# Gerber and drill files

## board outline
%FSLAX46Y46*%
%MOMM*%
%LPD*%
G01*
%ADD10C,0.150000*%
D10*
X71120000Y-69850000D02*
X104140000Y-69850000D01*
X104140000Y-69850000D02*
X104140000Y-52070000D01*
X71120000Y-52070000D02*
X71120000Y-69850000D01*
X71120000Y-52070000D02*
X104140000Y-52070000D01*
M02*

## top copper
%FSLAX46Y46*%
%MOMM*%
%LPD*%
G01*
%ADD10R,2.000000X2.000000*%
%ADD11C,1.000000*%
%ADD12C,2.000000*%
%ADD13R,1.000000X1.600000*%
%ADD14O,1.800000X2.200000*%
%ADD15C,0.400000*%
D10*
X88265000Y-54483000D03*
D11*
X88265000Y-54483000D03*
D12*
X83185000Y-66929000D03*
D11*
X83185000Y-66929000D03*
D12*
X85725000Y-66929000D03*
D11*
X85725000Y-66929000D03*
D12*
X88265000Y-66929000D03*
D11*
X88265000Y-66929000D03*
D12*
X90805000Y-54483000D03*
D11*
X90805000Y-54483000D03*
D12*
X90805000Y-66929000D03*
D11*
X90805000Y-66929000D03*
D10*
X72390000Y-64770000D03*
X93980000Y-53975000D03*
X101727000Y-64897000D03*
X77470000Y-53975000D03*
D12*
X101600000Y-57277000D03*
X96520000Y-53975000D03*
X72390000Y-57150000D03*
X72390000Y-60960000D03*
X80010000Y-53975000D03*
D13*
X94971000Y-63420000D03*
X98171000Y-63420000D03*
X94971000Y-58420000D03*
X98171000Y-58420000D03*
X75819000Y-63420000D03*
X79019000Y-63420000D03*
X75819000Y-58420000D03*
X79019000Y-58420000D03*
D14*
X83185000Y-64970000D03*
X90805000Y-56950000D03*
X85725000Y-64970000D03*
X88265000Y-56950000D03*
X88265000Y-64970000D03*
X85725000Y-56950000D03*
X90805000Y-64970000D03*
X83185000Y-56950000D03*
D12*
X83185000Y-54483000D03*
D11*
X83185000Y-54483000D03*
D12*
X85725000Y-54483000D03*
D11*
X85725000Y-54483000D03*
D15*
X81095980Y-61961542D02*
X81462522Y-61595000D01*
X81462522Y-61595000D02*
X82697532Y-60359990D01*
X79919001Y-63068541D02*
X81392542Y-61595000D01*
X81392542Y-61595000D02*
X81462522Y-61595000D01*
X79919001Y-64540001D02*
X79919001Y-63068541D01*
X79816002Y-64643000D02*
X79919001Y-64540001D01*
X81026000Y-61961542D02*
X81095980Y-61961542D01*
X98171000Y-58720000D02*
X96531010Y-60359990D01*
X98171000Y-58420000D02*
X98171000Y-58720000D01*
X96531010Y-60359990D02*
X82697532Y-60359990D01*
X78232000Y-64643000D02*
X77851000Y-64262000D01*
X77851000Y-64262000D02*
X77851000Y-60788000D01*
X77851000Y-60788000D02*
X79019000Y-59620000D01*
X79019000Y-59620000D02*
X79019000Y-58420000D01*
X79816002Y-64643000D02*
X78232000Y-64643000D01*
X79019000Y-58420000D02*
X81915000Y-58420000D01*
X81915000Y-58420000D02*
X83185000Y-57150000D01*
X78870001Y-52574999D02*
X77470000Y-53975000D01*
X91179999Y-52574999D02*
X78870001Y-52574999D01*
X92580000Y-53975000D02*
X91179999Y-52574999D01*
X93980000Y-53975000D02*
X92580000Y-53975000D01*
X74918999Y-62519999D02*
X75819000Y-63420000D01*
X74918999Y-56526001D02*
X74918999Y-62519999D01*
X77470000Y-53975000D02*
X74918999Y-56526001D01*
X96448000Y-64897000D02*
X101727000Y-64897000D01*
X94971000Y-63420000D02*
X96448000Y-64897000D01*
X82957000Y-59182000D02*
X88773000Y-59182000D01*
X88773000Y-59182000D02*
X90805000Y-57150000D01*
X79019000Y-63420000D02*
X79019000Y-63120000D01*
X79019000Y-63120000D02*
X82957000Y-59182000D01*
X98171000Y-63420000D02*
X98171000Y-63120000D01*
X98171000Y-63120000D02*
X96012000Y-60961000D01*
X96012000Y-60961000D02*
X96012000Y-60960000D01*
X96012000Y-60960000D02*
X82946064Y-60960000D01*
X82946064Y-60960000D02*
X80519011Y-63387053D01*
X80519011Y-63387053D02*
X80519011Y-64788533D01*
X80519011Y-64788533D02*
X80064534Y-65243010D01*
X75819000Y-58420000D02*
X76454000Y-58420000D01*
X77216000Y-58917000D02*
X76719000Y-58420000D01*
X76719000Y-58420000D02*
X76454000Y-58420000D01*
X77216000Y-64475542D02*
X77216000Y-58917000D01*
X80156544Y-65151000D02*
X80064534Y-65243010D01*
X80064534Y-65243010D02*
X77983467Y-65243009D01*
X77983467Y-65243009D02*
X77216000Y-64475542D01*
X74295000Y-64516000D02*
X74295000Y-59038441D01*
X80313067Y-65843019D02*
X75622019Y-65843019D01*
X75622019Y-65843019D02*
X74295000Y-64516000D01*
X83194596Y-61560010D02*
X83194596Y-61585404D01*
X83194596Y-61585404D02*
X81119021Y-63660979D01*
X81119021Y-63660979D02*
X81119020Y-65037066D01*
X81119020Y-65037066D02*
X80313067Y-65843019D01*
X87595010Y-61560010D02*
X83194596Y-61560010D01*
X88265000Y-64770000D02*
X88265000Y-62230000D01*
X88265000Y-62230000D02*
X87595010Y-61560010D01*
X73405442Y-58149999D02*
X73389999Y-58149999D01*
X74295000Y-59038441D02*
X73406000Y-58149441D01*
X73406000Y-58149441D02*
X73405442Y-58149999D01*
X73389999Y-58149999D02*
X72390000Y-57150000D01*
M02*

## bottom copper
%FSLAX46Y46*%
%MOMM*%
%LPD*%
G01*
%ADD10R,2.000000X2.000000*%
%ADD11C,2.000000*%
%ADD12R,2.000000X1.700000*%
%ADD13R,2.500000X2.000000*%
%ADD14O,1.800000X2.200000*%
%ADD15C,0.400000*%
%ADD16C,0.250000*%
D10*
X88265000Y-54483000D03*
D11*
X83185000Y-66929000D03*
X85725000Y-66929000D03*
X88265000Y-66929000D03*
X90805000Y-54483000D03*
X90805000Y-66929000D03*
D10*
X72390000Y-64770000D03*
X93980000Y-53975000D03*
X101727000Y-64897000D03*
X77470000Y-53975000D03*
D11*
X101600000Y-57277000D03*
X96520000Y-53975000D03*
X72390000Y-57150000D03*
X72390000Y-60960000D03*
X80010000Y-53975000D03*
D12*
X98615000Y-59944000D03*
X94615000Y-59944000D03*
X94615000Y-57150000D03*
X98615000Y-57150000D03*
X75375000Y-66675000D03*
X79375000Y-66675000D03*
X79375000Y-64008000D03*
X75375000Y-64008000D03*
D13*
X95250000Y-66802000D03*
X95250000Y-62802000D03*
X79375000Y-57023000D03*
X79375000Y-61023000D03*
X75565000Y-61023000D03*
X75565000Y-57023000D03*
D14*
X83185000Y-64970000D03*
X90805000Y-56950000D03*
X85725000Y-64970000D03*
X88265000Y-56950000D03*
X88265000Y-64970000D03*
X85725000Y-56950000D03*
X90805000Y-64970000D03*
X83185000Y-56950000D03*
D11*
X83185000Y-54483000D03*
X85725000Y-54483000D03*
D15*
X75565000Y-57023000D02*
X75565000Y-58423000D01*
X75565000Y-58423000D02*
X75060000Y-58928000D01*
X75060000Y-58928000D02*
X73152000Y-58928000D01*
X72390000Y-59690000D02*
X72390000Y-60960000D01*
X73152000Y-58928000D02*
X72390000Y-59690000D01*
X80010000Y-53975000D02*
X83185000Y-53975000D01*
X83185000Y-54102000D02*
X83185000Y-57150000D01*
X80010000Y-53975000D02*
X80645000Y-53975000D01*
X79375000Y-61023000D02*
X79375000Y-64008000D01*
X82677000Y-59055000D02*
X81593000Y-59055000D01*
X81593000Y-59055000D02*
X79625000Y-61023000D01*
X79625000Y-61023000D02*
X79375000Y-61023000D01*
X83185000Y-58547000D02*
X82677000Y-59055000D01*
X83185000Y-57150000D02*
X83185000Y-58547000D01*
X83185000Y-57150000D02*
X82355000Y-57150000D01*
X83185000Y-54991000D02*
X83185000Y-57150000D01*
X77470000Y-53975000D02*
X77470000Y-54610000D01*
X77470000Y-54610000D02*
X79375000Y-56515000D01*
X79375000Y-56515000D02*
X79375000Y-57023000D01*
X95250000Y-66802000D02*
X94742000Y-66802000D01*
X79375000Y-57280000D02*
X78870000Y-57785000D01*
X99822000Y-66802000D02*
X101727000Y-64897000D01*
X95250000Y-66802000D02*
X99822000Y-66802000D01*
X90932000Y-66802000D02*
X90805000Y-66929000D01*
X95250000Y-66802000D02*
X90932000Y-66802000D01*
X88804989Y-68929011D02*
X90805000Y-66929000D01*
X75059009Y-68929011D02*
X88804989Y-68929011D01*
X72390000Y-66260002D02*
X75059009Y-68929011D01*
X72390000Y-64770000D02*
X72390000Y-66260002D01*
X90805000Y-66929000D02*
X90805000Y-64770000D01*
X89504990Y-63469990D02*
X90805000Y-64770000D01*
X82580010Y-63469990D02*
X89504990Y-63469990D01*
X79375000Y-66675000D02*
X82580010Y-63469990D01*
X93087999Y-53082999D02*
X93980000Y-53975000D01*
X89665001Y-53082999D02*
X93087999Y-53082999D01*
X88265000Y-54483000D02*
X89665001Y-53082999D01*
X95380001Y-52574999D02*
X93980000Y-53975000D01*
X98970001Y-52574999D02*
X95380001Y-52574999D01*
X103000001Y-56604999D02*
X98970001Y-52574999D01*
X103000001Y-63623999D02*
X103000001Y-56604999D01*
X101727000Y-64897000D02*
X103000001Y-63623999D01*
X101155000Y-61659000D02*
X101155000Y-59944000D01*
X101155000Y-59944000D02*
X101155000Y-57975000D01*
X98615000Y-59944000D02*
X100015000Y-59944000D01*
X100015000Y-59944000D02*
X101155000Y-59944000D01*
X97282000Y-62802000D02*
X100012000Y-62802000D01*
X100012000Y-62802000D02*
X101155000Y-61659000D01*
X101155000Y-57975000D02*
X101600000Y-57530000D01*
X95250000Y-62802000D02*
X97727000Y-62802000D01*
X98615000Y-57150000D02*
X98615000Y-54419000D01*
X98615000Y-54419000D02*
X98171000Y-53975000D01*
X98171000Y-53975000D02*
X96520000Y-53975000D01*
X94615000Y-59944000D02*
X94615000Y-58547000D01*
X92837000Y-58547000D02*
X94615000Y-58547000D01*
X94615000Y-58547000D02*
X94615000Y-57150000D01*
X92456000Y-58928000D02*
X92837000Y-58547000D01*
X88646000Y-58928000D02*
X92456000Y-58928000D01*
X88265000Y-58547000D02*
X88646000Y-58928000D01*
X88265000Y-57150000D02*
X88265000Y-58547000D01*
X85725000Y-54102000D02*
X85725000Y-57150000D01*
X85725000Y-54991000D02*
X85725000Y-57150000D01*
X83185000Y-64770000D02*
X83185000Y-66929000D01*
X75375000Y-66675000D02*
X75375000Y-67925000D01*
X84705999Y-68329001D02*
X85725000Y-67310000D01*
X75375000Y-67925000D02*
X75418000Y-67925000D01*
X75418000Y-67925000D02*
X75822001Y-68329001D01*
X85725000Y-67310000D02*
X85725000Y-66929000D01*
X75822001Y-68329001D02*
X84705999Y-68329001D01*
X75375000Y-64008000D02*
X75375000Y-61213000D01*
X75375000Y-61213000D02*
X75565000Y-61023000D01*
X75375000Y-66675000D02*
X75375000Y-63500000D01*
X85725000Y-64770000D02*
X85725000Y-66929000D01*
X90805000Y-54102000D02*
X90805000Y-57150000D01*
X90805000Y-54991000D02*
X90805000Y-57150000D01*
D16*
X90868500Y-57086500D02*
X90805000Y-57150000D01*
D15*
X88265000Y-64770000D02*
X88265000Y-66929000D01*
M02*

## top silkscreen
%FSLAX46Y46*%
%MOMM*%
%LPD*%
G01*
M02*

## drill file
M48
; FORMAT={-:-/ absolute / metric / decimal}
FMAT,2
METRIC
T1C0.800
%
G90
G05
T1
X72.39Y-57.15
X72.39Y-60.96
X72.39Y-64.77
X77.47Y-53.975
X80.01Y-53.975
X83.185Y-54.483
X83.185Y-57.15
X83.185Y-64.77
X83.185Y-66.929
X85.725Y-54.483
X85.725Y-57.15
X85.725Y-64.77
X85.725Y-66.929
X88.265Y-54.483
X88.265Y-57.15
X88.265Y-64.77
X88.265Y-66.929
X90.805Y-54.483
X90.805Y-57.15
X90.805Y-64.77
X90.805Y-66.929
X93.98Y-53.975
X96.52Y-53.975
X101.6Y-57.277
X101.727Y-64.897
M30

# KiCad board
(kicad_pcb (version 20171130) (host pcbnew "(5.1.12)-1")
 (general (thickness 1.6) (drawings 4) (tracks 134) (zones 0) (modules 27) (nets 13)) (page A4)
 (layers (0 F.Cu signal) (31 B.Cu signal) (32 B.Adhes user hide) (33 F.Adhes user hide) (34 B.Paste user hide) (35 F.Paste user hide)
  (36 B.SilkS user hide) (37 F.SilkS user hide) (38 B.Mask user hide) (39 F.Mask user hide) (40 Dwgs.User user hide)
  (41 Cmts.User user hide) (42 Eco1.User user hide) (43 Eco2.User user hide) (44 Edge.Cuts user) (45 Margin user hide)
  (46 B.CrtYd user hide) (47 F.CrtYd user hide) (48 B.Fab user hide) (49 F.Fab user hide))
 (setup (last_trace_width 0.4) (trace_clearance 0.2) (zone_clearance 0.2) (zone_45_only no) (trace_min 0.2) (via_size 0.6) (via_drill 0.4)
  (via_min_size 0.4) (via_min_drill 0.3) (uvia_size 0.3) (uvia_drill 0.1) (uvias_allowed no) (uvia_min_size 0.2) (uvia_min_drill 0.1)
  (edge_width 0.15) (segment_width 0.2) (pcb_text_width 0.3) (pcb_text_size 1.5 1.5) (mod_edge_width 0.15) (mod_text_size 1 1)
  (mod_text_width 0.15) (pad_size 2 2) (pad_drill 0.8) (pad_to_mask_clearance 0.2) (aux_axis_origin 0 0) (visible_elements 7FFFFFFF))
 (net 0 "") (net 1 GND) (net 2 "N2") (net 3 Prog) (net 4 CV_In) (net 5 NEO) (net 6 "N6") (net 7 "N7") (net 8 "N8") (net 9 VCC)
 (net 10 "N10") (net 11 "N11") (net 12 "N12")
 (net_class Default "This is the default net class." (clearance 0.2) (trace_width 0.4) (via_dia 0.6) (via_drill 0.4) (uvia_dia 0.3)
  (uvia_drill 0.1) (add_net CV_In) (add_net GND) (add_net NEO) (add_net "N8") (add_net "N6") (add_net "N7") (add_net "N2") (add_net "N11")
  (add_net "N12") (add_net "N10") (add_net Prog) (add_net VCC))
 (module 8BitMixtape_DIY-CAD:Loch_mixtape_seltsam (layer F.Cu) (at 88.265 54.483)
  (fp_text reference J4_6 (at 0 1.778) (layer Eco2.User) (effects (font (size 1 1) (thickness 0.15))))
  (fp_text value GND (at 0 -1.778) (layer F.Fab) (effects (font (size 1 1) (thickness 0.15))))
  (pad 1 thru_hole rect (at 0 0) (size 2 2) (drill 0.8) (layers B.Cu B.Mask) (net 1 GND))
  (pad "" smd circle (at 0 0) (size 1 1) (layers F.Cu F.Paste F.Mask)))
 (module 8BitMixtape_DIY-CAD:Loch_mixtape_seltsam (layer F.Cu) (at 83.185 66.929)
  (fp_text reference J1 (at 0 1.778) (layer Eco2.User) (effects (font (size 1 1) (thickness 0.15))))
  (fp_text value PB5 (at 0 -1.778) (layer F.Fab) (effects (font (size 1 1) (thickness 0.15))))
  (pad 1 thru_hole circle (at 0 0) (size 2 2) (drill 0.8) (layers B.Cu B.Mask) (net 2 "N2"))
  (pad "" smd circle (at 0 0) (size 1 1) (layers F.Cu F.Paste F.Mask)))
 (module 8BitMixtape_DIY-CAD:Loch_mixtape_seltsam (layer F.Cu) (at 85.725 66.929)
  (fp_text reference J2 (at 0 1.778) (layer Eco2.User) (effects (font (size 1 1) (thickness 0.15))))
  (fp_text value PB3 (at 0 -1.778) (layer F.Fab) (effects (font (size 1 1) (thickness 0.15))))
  (pad 1 thru_hole circle (at 0 0) (size 2 2) (drill 0.8) (layers B.Cu B.Mask) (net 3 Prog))
  (pad "" smd circle (at 0 0) (size 1 1) (layers F.Cu F.Paste F.Mask)))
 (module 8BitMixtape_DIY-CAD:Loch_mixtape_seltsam (layer F.Cu) (at 88.265 66.929)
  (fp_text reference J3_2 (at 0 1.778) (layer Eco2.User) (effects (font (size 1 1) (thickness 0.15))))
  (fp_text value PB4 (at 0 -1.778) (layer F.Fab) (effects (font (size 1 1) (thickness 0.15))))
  (pad 1 thru_hole circle (at 0 0) (size 2 2) (drill 0.8) (layers B.Cu B.Mask) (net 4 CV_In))
  (pad "" smd circle (at 0 0) (size 1 1) (layers F.Cu F.Paste F.Mask)))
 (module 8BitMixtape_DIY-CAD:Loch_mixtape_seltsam (layer F.Cu) (at 90.805 54.483)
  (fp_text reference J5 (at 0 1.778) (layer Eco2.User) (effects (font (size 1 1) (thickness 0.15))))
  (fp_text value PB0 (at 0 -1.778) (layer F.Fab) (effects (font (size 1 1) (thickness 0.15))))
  (pad 1 thru_hole circle (at 0 0) (size 2 2) (drill 0.8) (layers B.Cu B.Mask) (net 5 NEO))
  (pad "" smd circle (at 0 0) (size 1 1) (layers F.Cu F.Paste F.Mask)))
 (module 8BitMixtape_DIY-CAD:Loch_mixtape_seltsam (layer F.Cu) (at 90.805 66.929)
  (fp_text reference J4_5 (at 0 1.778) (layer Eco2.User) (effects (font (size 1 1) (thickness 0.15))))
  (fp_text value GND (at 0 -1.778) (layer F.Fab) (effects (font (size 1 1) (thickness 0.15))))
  (pad 1 thru_hole circle (at 0 0) (size 2 2) (drill 0.8) (layers B.Cu B.Mask) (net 1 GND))
  (pad "" smd circle (at 0 0) (size 1 1) (layers F.Cu F.Paste F.Mask)))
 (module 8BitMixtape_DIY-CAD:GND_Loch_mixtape (layer F.Cu) (at 72.39 64.77)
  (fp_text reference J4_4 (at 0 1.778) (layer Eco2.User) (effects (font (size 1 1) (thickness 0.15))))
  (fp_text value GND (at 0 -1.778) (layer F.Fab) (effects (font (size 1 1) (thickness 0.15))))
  (pad 1 thru_hole rect (at 0 0) (size 2 2) (drill 0.8) (layers *.Cu *.Mask) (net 1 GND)))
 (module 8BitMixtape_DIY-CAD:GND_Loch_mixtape (layer F.Cu) (at 93.98 53.975)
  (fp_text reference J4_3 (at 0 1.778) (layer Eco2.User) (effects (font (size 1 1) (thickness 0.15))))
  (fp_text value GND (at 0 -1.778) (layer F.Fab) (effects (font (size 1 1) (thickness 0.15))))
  (pad 1 thru_hole rect (at 0 0) (size 2 2) (drill 0.8) (layers *.Cu *.Mask) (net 1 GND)))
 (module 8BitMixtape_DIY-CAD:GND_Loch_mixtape (layer F.Cu) (at 101.727 64.897)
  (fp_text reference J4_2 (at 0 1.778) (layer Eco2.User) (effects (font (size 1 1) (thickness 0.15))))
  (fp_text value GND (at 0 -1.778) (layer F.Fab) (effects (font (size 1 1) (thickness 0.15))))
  (pad 1 thru_hole rect (at 0 0) (size 2 2) (drill 0.8) (layers *.Cu *.Mask) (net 1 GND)))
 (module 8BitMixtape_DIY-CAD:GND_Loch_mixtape (layer F.Cu) (at 77.47 53.975)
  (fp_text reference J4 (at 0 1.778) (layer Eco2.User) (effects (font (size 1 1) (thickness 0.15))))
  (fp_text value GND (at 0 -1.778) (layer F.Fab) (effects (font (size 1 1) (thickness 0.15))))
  (pad 1 thru_hole rect (at 0 0) (size 2 2) (drill 0.8) (layers *.Cu *.Mask) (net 1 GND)))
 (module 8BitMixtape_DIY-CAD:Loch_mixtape (layer F.Cu) (at 101.6 57.277)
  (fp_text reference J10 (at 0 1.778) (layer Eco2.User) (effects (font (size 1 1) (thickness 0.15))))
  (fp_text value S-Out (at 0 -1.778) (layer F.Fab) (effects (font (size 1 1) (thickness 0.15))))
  (pad 1 thru_hole circle (at 0 0) (size 2 2) (drill 0.8) (layers *.Cu *.Mask) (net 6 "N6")))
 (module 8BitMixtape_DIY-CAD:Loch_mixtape (layer F.Cu) (at 96.52 53.975)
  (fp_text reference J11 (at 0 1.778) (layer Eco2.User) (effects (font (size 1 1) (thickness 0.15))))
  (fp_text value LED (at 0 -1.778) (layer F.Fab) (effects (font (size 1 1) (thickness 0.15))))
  (pad 1 thru_hole circle (at 0 0) (size 2 2) (drill 0.8) (layers *.Cu *.Mask) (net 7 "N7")))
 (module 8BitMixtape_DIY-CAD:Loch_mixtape (layer F.Cu) (at 72.39 57.15)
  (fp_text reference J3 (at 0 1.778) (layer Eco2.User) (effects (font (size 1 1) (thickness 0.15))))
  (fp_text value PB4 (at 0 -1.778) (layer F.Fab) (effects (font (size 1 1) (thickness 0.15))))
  (pad 1 thru_hole circle (at 0 0) (size 2 2) (drill 0.8) (layers *.Cu *.Mask) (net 4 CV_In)))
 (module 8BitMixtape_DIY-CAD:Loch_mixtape (layer F.Cu) (at 72.39 60.96)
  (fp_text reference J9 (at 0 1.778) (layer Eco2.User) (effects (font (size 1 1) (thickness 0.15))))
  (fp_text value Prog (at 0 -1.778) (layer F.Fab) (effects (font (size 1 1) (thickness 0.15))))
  (pad 1 thru_hole circle (at 0 0) (size 2 2) (drill 0.8) (layers *.Cu *.Mask) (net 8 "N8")))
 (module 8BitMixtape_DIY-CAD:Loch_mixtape (layer F.Cu) (at 80.01 53.975)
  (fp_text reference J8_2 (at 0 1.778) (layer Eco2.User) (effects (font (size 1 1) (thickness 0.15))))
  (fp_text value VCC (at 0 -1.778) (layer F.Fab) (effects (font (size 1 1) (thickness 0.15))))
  (pad 1 thru_hole circle (at 0 0) (size 2 2) (drill 0.8) (layers *.Cu *.Mask) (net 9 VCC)))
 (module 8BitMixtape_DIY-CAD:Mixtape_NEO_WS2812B (layer F.Cu) (at 96.571 60.92 270)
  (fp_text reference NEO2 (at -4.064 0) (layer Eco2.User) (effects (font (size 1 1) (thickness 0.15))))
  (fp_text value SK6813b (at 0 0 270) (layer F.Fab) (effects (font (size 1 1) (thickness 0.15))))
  (pad 3 smd rect (at 2.5 1.6 270) (size 1.6 1) (layers F.Cu F.Paste F.Mask) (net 1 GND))
  (pad 4 smd rect (at 2.5 -1.6 270) (size 1.6 1) (layers F.Cu F.Paste F.Mask) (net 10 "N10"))
  (pad 2 smd rect (at -2.5 1.6 270) (size 1.6 1) (layers F.Cu F.Paste F.Mask))
  (pad 1 smd rect (at -2.5 -1.6 270) (size 1.6 1) (layers F.Cu F.Paste F.Mask) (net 9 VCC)))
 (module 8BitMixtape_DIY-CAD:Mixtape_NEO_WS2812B (layer F.Cu) (at 77.419 60.92 270)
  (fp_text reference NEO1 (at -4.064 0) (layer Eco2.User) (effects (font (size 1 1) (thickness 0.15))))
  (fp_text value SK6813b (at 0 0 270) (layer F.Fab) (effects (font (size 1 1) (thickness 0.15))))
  (pad 3 smd rect (at 2.5 1.6 270) (size 1.6 1) (layers F.Cu F.Paste F.Mask) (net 1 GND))
  (pad 4 smd rect (at 2.5 -1.6 270) (size 1.6 1) (layers F.Cu F.Paste F.Mask) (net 5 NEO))
  (pad 2 smd rect (at -2.5 1.6 270) (size 1.6 1) (layers F.Cu F.Paste F.Mask) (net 10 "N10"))
  (pad 1 smd rect (at -2.5 -1.6 270) (size 1.6 1) (layers F.Cu F.Paste F.Mask) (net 9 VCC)))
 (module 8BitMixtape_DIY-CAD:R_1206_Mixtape (layer B.Cu) (at 96.615 59.944 180)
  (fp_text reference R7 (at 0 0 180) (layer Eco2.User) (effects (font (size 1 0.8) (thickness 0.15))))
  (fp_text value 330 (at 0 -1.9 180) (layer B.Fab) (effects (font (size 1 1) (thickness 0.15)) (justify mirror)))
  (pad 1 smd rect (at -2 0 180) (size 2 1.7) (layers B.Cu B.Paste B.Mask) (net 6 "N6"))
  (pad 2 smd rect (at 2 0 180) (size 2 1.7) (layers B.Cu B.Paste B.Mask) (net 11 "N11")))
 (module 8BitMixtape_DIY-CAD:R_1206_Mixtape (layer B.Cu) (at 96.615 57.15)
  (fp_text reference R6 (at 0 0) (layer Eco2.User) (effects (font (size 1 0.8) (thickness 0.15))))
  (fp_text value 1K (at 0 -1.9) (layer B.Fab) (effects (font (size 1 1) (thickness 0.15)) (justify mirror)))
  (pad 1 smd rect (at -2 0) (size 2 1.7) (layers B.Cu B.Paste B.Mask) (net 11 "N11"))
  (pad 2 smd rect (at 2 0) (size 2 1.7) (layers B.Cu B.Paste B.Mask) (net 7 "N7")))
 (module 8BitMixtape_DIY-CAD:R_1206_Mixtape (layer B.Cu) (at 77.375 66.675)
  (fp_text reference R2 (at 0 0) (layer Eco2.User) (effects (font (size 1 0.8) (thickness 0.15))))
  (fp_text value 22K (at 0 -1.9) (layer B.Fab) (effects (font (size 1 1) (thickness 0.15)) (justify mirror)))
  (pad 1 smd rect (at -2 0) (size 2 1.7) (layers B.Cu B.Paste B.Mask) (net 3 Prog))
  (pad 2 smd rect (at 2 0) (size 2 1.7) (layers B.Cu B.Paste B.Mask) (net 1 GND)))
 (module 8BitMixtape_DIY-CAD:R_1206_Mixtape (layer B.Cu) (at 77.375 64.008 180)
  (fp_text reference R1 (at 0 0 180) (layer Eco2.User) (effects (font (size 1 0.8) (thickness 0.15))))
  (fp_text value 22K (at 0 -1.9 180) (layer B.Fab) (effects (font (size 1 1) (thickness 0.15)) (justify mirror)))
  (pad 1 smd rect (at -2 0 180) (size 2 1.7) (layers B.Cu B.Paste B.Mask) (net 9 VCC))
  (pad 2 smd rect (at 2 0 180) (size 2 1.7) (layers B.Cu B.Paste B.Mask) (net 3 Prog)))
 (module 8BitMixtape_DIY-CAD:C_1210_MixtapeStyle (layer B.Cu) (at 95.25 64.802 90)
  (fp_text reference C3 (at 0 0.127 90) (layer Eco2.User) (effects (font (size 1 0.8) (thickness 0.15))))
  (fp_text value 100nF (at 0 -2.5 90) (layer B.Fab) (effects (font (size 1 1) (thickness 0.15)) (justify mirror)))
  (pad 1 smd rect (at -2 0 90) (size 2 2.5) (layers B.Cu B.Paste B.Mask) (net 1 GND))
  (pad 2 smd rect (at 2 0 90) (size 2 2.5) (layers B.Cu B.Paste B.Mask) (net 6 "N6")))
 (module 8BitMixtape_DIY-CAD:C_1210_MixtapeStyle (layer B.Cu) (at 79.375 59.023 270)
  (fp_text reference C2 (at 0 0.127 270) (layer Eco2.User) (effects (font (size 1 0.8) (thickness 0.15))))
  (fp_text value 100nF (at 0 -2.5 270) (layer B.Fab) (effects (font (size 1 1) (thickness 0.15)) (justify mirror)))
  (pad 1 smd rect (at -2 0 270) (size 2 2.5) (layers B.Cu B.Paste B.Mask) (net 1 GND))
  (pad 2 smd rect (at 2 0 270) (size 2 2.5) (layers B.Cu B.Paste B.Mask) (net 9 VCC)))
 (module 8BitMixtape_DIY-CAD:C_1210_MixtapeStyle (layer B.Cu) (at 75.565 59.023 90)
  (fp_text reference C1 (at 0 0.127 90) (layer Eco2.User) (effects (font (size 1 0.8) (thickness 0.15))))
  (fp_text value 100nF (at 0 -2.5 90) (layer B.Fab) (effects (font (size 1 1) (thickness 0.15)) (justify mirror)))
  (pad 1 smd rect (at -2 0 90) (size 2 2.5) (layers B.Cu B.Paste B.Mask) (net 3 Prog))
  (pad 2 smd rect (at 2 0 90) (size 2 2.5) (layers B.Cu B.Paste B.Mask) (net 8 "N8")))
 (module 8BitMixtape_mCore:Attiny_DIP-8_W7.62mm (layer F.Cu) (at 83.185 64.77 90)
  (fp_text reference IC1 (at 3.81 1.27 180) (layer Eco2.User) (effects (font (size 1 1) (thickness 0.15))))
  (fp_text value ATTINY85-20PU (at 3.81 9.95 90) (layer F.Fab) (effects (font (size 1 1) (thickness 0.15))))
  (pad 1 thru_hole oval (at 0 0 90) (size 2.2 1.8) (drill 0.8 (offset -0.2 0)) (layers *.Cu *.Mask) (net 2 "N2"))
  (pad 5 thru_hole oval (at 7.62 7.62 90) (size 2.2 1.8) (drill 0.8 (offset 0.2 0)) (layers *.Cu *.Mask) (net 5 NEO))
  (pad 2 thru_hole oval (at 0 2.54 90) (size 2.2 1.8) (drill 0.8 (offset -0.2 0)) (layers *.Cu *.Mask) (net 3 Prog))
  (pad 6 thru_hole oval (at 7.62 5.08 90) (size 2.2 1.8) (drill 0.8 (offset 0.2 0)) (layers *.Cu *.Mask) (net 11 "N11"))
  (pad 3 thru_hole oval (at 0 5.08 90) (size 2.2 1.8) (drill 0.8 (offset -0.2 0)) (layers *.Cu *.Mask) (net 4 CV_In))
  (pad 7 thru_hole oval (at 7.62 2.54 90) (size 2.2 1.8) (drill 0.8 (offset 0.2 0)) (layers *.Cu *.Mask) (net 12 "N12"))
  (pad 4 thru_hole oval (at 0 7.62 90) (size 2.2 1.8) (drill 0.8 (offset -0.2 0)) (layers *.Cu *.Mask) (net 1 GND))
  (pad 8 thru_hole oval (at 7.62 0 90) (size 2.2 1.8) (drill 0.8 (offset 0.2 0)) (layers *.Cu *.Mask) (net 9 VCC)))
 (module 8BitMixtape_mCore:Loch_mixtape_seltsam (layer F.Cu) (at 83.185 54.483)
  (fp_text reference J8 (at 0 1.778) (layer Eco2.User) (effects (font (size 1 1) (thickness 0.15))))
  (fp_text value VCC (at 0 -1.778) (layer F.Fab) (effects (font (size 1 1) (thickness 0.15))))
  (pad 1 thru_hole circle (at 0 0) (size 2 2) (drill 0.8) (layers B.Cu B.Mask) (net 9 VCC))
  (pad "" smd circle (at 0 0) (size 1 1) (layers F.Cu F.Paste F.Mask)))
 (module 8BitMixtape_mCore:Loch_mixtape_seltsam (layer F.Cu) (at 85.725 54.483)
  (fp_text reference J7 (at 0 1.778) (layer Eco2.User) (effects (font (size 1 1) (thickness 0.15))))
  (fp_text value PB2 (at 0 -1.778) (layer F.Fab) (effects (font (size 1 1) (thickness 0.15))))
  (pad 1 thru_hole circle (at 0 0) (size 2 2) (drill 0.8) (layers B.Cu B.Mask) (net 12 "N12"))
  (pad "" smd circle (at 0 0) (size 1 1) (layers F.Cu F.Paste F.Mask)))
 (gr_line (start 71.12 69.85) (end 104.14 69.85) (layer Edge.Cuts) (width 0.15))
 (gr_line (start 104.14 69.85) (end 104.14 52.07) (layer Edge.Cuts) (width 0.15))
 (gr_line (start 71.12 52.07) (end 71.12 69.85) (layer Edge.Cuts) (width 0.15))
 (gr_line (start 71.12 52.07) (end 104.14 52.07) (layer Edge.Cuts) (width 0.15))
 (segment (start 75.565 57.023) (end 75.565 58.423) (width 0.4) (layer B.Cu) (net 8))
 (segment (start 75.565 58.423) (end 75.06 58.928) (width 0.4) (layer B.Cu) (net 8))
 (segment (start 75.06 58.928) (end 73.152 58.928) (width 0.4) (layer B.Cu) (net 8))
 (segment (start 72.39 59.69) (end 72.39 60.96) (width 0.4) (layer B.Cu) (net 8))
 (segment (start 73.152 58.928) (end 72.39 59.69) (width 0.4) (layer B.Cu) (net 8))
 (segment (start 81.09598 61.961542) (end 81.462522 61.595) (width 0.4) (layer F.Cu) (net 9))
 (segment (start 81.462522 61.595) (end 82.697532 60.35999) (width 0.4) (layer F.Cu) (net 9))
 (segment (start 79.919001 63.068541) (end 81.392542 61.595) (width 0.4) (layer F.Cu) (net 9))
 (segment (start 81.392542 61.595) (end 81.462522 61.595) (width 0.4) (layer F.Cu) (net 9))
 (segment (start 79.919001 64.540001) (end 79.919001 63.068541) (width 0.4) (layer F.Cu) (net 9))
 (segment (start 79.816002 64.643) (end 79.919001 64.540001) (width 0.4) (layer F.Cu) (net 9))
 (segment (start 81.026 61.961542) (end 81.09598 61.961542) (width 0.4) (layer F.Cu) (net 9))
 (segment (start 98.171 58.72) (end 96.53101 60.35999) (width 0.4) (layer F.Cu) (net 9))
 (segment (start 98.171 58.42) (end 98.171 58.72) (width 0.4) (layer F.Cu) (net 9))
 (segment (start 96.53101 60.35999) (end 82.697532 60.35999) (width 0.4) (layer F.Cu) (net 9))
 (segment (start 78.232 64.643) (end 77.851 64.262) (width 0.4) (layer F.Cu) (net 9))
 (segment (start 77.851 64.262) (end 77.851 60.788) (width 0.4) (layer F.Cu) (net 9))
 (segment (start 77.851 60.788) (end 79.019 59.62) (width 0.4) (layer F.Cu) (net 9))
 (segment (start 79.019 59.62) (end 79.019 58.42) (width 0.4) (layer F.Cu) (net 9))
 (segment (start 79.816002 64.643) (end 78.232 64.643) (width 0.4) (layer F.Cu) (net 9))
 (segment (start 79.019 58.42) (end 81.915 58.42) (width 0.4) (layer F.Cu) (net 9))
 (segment (start 81.915 58.42) (end 83.185 57.15) (width 0.4) (layer F.Cu) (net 9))
 (segment (start 80.01 53.975) (end 83.185 53.975) (width 0.4) (layer B.Cu) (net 9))
 (segment (start 83.185 54.102) (end 83.185 57.15) (width 0.4) (layer B.Cu) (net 9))
 (segment (start 80.01 53.975) (end 80.645 53.975) (width 0.4) (layer B.Cu) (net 9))
 (segment (start 79.375 61.023) (end 79.375 64.008) (width 0.4) (layer B.Cu) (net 9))
 (segment (start 82.677 59.055) (end 81.593 59.055) (width 0.4) (layer B.Cu) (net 9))
 (segment (start 81.593 59.055) (end 79.625 61.023) (width 0.4) (layer B.Cu) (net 9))
 (segment (start 79.625 61.023) (end 79.375 61.023) (width 0.4) (layer B.Cu) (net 9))
 (segment (start 83.185 58.547) (end 82.677 59.055) (width 0.4) (layer B.Cu) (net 9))
 (segment (start 83.185 57.15) (end 83.185 58.547) (width 0.4) (layer B.Cu) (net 9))
 (segment (start 83.185 57.15) (end 82.355 57.15) (width 0.4) (layer B.Cu) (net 9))
 (segment (start 83.185 54.991) (end 83.185 57.15) (width 0.4) (layer B.Cu) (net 9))
 (segment (start 77.47 53.975) (end 77.47 54.61) (width 0.4) (layer B.Cu) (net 1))
 (segment (start 77.47 54.61) (end 79.375 56.515) (width 0.4) (layer B.Cu) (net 1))
 (segment (start 79.375 56.515) (end 79.375 57.023) (width 0.4) (layer B.Cu) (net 1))
 (segment (start 95.25 66.802) (end 94.742 66.802) (width 0.4) (layer B.Cu) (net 1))
 (segment (start 79.375 57.28) (end 78.87 57.785) (width 0.4) (layer B.Cu) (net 1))
 (segment (start 78.870001 52.574999) (end 77.47 53.975) (width 0.4) (layer F.Cu) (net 1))
 (segment (start 91.179999 52.574999) (end 78.870001 52.574999) (width 0.4) (layer F.Cu) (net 1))
 (segment (start 92.58 53.975) (end 91.179999 52.574999) (width 0.4) (layer F.Cu) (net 1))
 (segment (start 93.98 53.975) (end 92.58 53.975) (width 0.4) (layer F.Cu) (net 1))
 (segment (start 74.918999 62.519999) (end 75.819 63.42) (width 0.4) (layer F.Cu) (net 1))
 (segment (start 74.918999 56.526001) (end 74.918999 62.519999) (width 0.4) (layer F.Cu) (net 1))
 (segment (start 77.47 53.975) (end 74.918999 56.526001) (width 0.4) (layer F.Cu) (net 1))
 (segment (start 96.448 64.897) (end 101.727 64.897) (width 0.4) (layer F.Cu) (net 1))
 (segment (start 94.971 63.42) (end 96.448 64.897) (width 0.4) (layer F.Cu) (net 1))
 (segment (start 99.822 66.802) (end 101.727 64.897) (width 0.4) (layer B.Cu) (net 1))
 (segment (start 95.25 66.802) (end 99.822 66.802) (width 0.4) (layer B.Cu) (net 1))
 (segment (start 90.932 66.802) (end 90.805 66.929) (width 0.4) (layer B.Cu) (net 1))
 (segment (start 95.25 66.802) (end 90.932 66.802) (width 0.4) (layer B.Cu) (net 1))
 (segment (start 88.804989 68.929011) (end 90.805 66.929) (width 0.4) (layer B.Cu) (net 1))
 (segment (start 75.059009 68.929011) (end 88.804989 68.929011) (width 0.4) (layer B.Cu) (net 1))
 (segment (start 72.39 66.260002) (end 75.059009 68.929011) (width 0.4) (layer B.Cu) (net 1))
 (segment (start 72.39 64.77) (end 72.39 66.260002) (width 0.4) (layer B.Cu) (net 1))
 (segment (start 90.805 66.929) (end 90.805 64.77) (width 0.4) (layer B.Cu) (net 1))
 (segment (start 89.50499 63.46999) (end 90.805 64.77) (width 0.4) (layer B.Cu) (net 1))
 (segment (start 82.58001 63.46999) (end 89.50499 63.46999) (width 0.4) (layer B.Cu) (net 1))
 (segment (start 79.375 66.675) (end 82.58001 63.46999) (width 0.4) (layer B.Cu) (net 1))
 (segment (start 93.087999 53.082999) (end 93.98 53.975) (width 0.4) (layer B.Cu) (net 1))
 (segment (start 89.665001 53.082999) (end 93.087999 53.082999) (width 0.4) (layer B.Cu) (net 1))
 (segment (start 88.265 54.483) (end 89.665001 53.082999) (width 0.4) (layer B.Cu) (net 1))
 (segment (start 95.380001 52.574999) (end 93.98 53.975) (width 0.4) (layer B.Cu) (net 1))
 (segment (start 98.970001 52.574999) (end 95.380001 52.574999) (width 0.4) (layer B.Cu) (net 1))
 (segment (start 103.000001 56.604999) (end 98.970001 52.574999) (width 0.4) (layer B.Cu) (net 1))
 (segment (start 103.000001 63.623999) (end 103.000001 56.604999) (width 0.4) (layer B.Cu) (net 1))
 (segment (start 101.727 64.897) (end 103.000001 63.623999) (width 0.4) (layer B.Cu) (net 1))
 (segment (start 101.155 61.659) (end 101.155 59.944) (width 0.4) (layer B.Cu) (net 6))
 (segment (start 101.155 59.944) (end 101.155 57.975) (width 0.4) (layer B.Cu) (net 6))
 (segment (start 98.615 59.944) (end 100.015 59.944) (width 0.4) (layer B.Cu) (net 6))
 (segment (start 100.015 59.944) (end 101.155 59.944) (width 0.4) (layer B.Cu) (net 6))
 (segment (start 97.282 62.802) (end 100.012 62.802) (width 0.4) (layer B.Cu) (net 6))
 (segment (start 100.012 62.802) (end 101.155 61.659) (width 0.4) (layer B.Cu) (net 6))
 (segment (start 101.155 57.975) (end 101.6 57.53) (width 0.4) (layer B.Cu) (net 6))
 (segment (start 95.25 62.802) (end 97.727 62.802) (width 0.4) (layer B.Cu) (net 6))
 (segment (start 98.615 57.15) (end 98.615 54.419) (width 0.4) (layer B.Cu) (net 7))
 (segment (start 98.615 54.419) (end 98.171 53.975) (width 0.4) (layer B.Cu) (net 7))
 (segment (start 98.171 53.975) (end 96.52 53.975) (width 0.4) (layer B.Cu) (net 7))
 (segment (start 94.615 59.944) (end 94.615 58.547) (width 0.4) (layer B.Cu) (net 11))
 (segment (start 92.837 58.547) (end 94.615 58.547) (width 0.4) (layer B.Cu) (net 11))
 (segment (start 94.615 58.547) (end 94.615 57.15) (width 0.4) (layer B.Cu) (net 11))
 (segment (start 92.456 58.928) (end 92.837 58.547) (width 0.4) (layer B.Cu) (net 11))
 (segment (start 88.646 58.928) (end 92.456 58.928) (width 0.4) (layer B.Cu) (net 11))
 (segment (start 88.265 58.547) (end 88.646 58.928) (width 0.4) (layer B.Cu) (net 11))
 (segment (start 88.265 57.15) (end 88.265 58.547) (width 0.4) (layer B.Cu) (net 11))
 (segment (start 85.725 54.102) (end 85.725 57.15) (width 0.4) (layer B.Cu) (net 12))
 (segment (start 85.725 54.991) (end 85.725 57.15) (width 0.4) (layer B.Cu) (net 12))
 (segment (start 83.185 64.77) (end 83.185 66.929) (width 0.4) (layer B.Cu) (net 2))
 (segment (start 75.375 66.675) (end 75.375 67.925) (width 0.4) (layer B.Cu) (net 3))
 (segment (start 84.705999 68.329001) (end 85.725 67.31) (width 0.4) (layer B.Cu) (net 3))
 (segment (start 75.375 67.925) (end 75.418 67.925) (width 0.4) (layer B.Cu) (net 3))
 (segment (start 75.418 67.925) (end 75.822001 68.329001) (width 0.4) (layer B.Cu) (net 3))
 (segment (start 85.725 67.31) (end 85.725 66.929) (width 0.4) (layer B.Cu) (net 3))
 (segment (start 75.822001 68.329001) (end 84.705999 68.329001) (width 0.4) (layer B.Cu) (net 3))
 (segment (start 75.375 64.008) (end 75.375 61.213) (width 0.4) (layer B.Cu) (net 3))
 (segment (start 75.375 61.213) (end 75.565 61.023) (width 0.4) (layer B.Cu) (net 3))
 (segment (start 75.375 66.675) (end 75.375 63.5) (width 0.4) (layer B.Cu) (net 3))
 (segment (start 85.725 64.77) (end 85.725 66.929) (width 0.4) (layer B.Cu) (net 3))
 (segment (start 82.957 59.182) (end 88.773 59.182) (width 0.4) (layer F.Cu) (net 5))
 (segment (start 88.773 59.182) (end 90.805 57.15) (width 0.4) (layer F.Cu) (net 5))
 (segment (start 79.019 63.42) (end 79.019 63.12) (width 0.4) (layer F.Cu) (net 5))
 (segment (start 79.019 63.12) (end 82.957 59.182) (width 0.4) (layer F.Cu) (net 5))
 (segment (start 90.805 54.102) (end 90.805 57.15) (width 0.4) (layer B.Cu) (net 5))
 (segment (start 90.805 54.991) (end 90.805 57.15) (width 0.4) (layer B.Cu) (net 5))
 (segment (start 90.8685 57.0865) (end 90.805 57.15) (width 0.25) (layer B.Cu) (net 5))
 (segment (start 98.171 63.42) (end 98.171 63.12) (width 0.4) (layer F.Cu) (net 10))
 (segment (start 98.171 63.12) (end 96.012 60.961) (width 0.4) (layer F.Cu) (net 10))
 (segment (start 96.012 60.961) (end 96.012 60.96) (width 0.4) (layer F.Cu) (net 10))
 (segment (start 96.012 60.96) (end 82.946064 60.96) (width 0.4) (layer F.Cu) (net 10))
 (segment (start 82.946064 60.96) (end 80.519011 63.387053) (width 0.4) (layer F.Cu) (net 10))
 (segment (start 80.519011 63.387053) (end 80.519011 64.788533) (width 0.4) (layer F.Cu) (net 10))
 (segment (start 80.519011 64.788533) (end 80.064534 65.24301) (width 0.4) (layer F.Cu) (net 10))
 (segment (start 75.819 58.42) (end 76.454 58.42) (width 0.4) (layer F.Cu) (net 10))
 (segment (start 77.216 58.917) (end 76.719 58.42) (width 0.4) (layer F.Cu) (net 10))
 (segment (start 76.719 58.42) (end 76.454 58.42) (width 0.4) (layer F.Cu) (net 10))
 (segment (start 77.216 64.475542) (end 77.216 58.917) (width 0.4) (layer F.Cu) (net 10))
 (segment (start 80.156544 65.151) (end 80.064534 65.24301) (width 0.4) (layer F.Cu) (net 10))
 (segment (start 80.064534 65.24301) (end 77.983467 65.243009) (width 0.4) (layer F.Cu) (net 10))
 (segment (start 77.983467 65.243009) (end 77.216 64.475542) (width 0.4) (layer F.Cu) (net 10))
 (segment (start 74.295 64.516) (end 74.295 59.038441) (width 0.4) (layer F.Cu) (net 4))
 (segment (start 80.313067 65.843019) (end 75.622019 65.843019) (width 0.4) (layer F.Cu) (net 4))
 (segment (start 75.622019 65.843019) (end 74.295 64.516) (width 0.4) (layer F.Cu) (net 4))
 (segment (start 83.194596 61.56001) (end 83.194596 61.585404) (width 0.4) (layer F.Cu) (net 4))
 (segment (start 83.194596 61.585404) (end 81.119021 63.660979) (width 0.4) (layer F.Cu) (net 4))
 (segment (start 81.119021 63.660979) (end 81.11902 65.037066) (width 0.4) (layer F.Cu) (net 4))
 (segment (start 81.11902 65.037066) (end 80.313067 65.843019) (width 0.4) (layer F.Cu) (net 4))
 (segment (start 87.59501 61.56001) (end 83.194596 61.56001) (width 0.4) (layer F.Cu) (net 4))
 (segment (start 88.265 64.77) (end 88.265 62.23) (width 0.4) (layer F.Cu) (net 4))
 (segment (start 88.265 62.23) (end 87.59501 61.56001) (width 0.4) (layer F.Cu) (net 4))
 (segment (start 73.405442 58.149999) (end 73.389999 58.149999) (width 0.4) (layer F.Cu) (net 4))
 (segment (start 74.295 59.038441) (end 73.406 58.149441) (width 0.4) (layer F.Cu) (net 4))
 (segment (start 73.406 58.149441) (end 73.405442 58.149999) (width 0.4) (layer F.Cu) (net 4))
 (segment (start 73.389999 58.149999) (end 72.39 57.15) (width 0.4) (layer F.Cu) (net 4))
 (segment (start 88.265 64.77) (end 88.265 66.929) (width 0.4) (layer B.Cu) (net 4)))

